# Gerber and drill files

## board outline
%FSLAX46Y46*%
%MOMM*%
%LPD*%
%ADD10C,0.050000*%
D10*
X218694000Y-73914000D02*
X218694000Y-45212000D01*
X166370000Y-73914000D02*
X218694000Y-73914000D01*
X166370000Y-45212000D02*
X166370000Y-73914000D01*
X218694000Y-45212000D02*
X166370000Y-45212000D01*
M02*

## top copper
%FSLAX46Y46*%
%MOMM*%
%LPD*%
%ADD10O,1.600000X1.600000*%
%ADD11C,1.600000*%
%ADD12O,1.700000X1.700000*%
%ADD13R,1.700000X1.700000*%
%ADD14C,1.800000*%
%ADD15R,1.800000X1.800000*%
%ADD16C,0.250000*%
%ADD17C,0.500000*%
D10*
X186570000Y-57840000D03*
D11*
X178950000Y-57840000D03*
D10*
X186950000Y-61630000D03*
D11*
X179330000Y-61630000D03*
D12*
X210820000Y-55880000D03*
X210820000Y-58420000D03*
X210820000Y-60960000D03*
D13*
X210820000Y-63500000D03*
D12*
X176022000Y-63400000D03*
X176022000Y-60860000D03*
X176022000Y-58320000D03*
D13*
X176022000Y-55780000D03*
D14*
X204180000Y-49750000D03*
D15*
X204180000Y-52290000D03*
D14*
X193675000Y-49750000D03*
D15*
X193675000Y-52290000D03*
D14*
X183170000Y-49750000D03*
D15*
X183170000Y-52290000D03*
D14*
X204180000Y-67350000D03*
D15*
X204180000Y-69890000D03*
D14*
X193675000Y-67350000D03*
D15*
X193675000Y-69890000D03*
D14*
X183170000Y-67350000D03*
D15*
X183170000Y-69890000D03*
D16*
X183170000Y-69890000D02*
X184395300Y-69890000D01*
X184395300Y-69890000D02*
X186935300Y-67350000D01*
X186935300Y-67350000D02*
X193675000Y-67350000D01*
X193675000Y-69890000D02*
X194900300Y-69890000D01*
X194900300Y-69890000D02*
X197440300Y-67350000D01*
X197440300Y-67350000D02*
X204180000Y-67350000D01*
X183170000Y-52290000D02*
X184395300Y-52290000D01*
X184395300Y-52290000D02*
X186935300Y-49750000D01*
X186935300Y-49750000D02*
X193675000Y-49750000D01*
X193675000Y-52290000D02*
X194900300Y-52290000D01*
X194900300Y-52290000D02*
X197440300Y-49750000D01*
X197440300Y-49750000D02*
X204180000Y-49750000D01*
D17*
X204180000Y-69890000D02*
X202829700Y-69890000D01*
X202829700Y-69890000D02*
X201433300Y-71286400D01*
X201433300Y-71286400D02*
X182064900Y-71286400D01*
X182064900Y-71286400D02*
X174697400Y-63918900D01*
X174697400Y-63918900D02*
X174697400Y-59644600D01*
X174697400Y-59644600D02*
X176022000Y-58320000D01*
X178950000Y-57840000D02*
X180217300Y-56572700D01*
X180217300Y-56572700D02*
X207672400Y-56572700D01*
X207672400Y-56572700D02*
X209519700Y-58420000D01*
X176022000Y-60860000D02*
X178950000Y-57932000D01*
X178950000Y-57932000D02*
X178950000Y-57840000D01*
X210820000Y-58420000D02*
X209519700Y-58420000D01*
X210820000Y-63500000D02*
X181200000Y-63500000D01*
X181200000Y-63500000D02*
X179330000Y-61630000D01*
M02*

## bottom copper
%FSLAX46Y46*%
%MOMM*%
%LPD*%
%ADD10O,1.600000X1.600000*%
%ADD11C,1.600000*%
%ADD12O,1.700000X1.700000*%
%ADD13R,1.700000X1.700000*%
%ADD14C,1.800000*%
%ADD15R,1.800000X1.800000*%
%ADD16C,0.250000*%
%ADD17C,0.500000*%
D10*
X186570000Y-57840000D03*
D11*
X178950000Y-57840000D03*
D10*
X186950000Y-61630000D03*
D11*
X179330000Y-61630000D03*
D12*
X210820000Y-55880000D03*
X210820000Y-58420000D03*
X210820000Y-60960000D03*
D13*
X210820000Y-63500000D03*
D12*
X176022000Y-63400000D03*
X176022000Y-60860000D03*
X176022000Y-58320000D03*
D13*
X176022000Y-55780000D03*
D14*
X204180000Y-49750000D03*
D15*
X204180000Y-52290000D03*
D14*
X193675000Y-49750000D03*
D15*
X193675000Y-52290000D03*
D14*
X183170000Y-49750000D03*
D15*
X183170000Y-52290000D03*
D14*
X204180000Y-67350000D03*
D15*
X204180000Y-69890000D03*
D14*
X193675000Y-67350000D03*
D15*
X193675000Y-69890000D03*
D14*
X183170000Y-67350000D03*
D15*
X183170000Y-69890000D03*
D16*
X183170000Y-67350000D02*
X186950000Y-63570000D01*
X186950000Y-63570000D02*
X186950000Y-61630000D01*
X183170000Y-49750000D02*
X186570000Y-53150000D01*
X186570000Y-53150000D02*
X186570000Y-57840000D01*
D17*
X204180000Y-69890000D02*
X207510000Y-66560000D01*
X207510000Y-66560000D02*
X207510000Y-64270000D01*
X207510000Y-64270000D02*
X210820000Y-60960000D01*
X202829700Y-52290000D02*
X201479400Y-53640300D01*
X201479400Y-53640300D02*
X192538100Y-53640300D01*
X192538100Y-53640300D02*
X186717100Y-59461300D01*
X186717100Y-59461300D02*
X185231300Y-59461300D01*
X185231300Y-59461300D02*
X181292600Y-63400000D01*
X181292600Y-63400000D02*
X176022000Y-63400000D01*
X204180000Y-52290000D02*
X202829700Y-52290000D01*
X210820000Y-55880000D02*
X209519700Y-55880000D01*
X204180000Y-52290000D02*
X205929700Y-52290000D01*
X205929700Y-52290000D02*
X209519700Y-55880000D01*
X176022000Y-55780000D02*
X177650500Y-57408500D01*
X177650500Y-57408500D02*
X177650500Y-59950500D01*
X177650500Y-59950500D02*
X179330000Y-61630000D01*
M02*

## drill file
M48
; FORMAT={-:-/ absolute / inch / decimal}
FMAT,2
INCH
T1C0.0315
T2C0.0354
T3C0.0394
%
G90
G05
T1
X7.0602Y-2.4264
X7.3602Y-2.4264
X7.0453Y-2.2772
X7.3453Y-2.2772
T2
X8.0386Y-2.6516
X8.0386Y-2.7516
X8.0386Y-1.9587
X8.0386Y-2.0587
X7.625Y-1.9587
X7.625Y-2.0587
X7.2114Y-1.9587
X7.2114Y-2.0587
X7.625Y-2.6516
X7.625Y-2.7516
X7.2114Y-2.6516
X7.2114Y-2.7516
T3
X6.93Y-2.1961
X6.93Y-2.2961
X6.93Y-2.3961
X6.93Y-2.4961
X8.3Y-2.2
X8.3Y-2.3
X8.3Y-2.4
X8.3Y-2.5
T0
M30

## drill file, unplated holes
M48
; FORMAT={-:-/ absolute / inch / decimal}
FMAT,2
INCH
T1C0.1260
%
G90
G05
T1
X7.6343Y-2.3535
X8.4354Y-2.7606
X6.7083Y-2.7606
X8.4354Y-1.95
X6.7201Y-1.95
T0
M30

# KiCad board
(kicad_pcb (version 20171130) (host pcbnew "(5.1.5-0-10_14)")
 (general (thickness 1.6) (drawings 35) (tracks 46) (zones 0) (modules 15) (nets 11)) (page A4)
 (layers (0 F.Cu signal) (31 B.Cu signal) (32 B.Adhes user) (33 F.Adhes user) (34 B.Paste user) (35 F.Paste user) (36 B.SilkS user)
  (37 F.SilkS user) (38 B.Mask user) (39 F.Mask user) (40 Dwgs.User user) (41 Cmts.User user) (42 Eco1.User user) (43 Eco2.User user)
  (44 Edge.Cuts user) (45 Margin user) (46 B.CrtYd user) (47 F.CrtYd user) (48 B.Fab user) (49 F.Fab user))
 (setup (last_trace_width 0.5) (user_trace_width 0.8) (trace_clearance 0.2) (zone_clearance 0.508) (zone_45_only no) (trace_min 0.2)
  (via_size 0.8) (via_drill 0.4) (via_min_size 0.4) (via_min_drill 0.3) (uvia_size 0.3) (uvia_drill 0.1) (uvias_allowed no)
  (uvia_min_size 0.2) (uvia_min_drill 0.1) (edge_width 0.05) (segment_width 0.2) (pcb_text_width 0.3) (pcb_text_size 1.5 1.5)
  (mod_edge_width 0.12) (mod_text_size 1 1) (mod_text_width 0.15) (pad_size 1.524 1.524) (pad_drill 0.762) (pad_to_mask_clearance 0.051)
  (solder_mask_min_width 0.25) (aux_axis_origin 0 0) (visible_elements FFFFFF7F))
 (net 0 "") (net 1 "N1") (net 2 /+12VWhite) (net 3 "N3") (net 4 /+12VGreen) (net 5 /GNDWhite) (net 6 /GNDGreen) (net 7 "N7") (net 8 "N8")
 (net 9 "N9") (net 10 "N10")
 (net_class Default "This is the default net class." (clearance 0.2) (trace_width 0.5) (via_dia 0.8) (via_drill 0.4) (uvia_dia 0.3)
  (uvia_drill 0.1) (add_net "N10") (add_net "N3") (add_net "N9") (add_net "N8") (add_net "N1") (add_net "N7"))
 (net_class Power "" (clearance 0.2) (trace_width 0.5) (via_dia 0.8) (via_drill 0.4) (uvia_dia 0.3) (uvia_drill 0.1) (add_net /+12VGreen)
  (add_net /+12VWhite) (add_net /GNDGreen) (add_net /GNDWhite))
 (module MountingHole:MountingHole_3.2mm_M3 (layer F.Cu) (at 193.91 59.78)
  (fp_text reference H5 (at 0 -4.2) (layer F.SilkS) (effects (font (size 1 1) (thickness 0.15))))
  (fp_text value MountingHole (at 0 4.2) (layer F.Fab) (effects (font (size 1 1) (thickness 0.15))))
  (pad 1 np_thru_hole circle (at 0 0) (size 3.2 3.2) (drill 3.2) (layers *.Cu *.Mask)))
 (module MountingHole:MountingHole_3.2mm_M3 (layer F.Cu) (at 214.26 70.12)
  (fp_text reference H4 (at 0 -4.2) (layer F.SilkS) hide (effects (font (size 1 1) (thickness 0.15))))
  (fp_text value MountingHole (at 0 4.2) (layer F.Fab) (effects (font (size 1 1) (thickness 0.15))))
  (pad 1 np_thru_hole circle (at 0 0) (size 3.2 3.2) (drill 3.2) (layers *.Cu *.Mask)))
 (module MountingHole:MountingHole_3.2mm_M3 (layer F.Cu) (at 170.39 70.12)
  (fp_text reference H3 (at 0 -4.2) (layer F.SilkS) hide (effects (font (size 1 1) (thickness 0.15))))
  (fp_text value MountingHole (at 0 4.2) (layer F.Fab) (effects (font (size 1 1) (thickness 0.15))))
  (pad 1 np_thru_hole circle (at 0 0) (size 3.2 3.2) (drill 3.2) (layers *.Cu *.Mask)))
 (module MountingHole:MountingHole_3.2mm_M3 (layer F.Cu) (at 214.26 49.53)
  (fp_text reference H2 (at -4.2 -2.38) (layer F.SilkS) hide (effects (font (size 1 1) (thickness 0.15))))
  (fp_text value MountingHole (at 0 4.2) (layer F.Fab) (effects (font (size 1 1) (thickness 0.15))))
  (pad 1 np_thru_hole circle (at 0 0) (size 3.2 3.2) (drill 3.2) (layers *.Cu *.Mask)))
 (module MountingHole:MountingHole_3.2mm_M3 (layer F.Cu) (at 170.69 49.53)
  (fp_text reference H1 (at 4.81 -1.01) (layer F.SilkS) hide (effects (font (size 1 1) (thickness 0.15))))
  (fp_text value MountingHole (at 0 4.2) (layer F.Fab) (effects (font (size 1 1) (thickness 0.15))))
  (pad 1 np_thru_hole circle (at 0 0) (size 3.2 3.2) (drill 3.2) (layers *.Cu *.Mask)))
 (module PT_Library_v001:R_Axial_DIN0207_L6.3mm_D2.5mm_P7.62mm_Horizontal (layer B.Cu) (at 178.95 57.84)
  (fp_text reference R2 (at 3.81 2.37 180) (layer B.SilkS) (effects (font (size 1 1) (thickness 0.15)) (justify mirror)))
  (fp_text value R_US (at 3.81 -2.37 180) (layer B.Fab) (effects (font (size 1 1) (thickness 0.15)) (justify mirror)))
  (pad 2 thru_hole oval (at 7.62 0) (size 1.6 1.6) (drill 0.8) (layers *.Cu *.Mask) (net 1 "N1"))
  (pad 1 thru_hole circle (at 0 0) (size 1.6 1.6) (drill 0.8) (layers *.Cu *.Mask) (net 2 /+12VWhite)))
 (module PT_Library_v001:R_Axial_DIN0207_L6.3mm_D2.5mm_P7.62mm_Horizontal (layer B.Cu) (at 179.33 61.63)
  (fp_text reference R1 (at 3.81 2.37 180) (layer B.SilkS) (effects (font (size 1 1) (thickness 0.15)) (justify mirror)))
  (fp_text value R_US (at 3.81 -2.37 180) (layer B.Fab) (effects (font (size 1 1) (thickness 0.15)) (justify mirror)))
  (pad 2 thru_hole oval (at 7.62 0) (size 1.6 1.6) (drill 0.8) (layers *.Cu *.Mask) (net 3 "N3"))
  (pad 1 thru_hole circle (at 0 0) (size 1.6 1.6) (drill 0.8) (layers *.Cu *.Mask) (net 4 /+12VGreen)))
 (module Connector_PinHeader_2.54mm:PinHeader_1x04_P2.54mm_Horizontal (layer B.Cu) (at 210.82 63.5)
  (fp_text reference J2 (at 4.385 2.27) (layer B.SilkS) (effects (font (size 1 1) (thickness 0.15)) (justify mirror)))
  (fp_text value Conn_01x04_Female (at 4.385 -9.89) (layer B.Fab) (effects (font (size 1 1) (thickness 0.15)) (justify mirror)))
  (pad 4 thru_hole oval (at 0 -7.62) (size 1.7 1.7) (drill 1) (layers *.Cu *.Mask) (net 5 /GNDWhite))
  (pad 3 thru_hole oval (at 0 -5.08) (size 1.7 1.7) (drill 1) (layers *.Cu *.Mask) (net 2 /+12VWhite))
  (pad 2 thru_hole oval (at 0 -2.54) (size 1.7 1.7) (drill 1) (layers *.Cu *.Mask) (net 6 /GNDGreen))
  (pad 1 thru_hole rect (at 0 0) (size 1.7 1.7) (drill 1) (layers *.Cu *.Mask) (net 4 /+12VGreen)))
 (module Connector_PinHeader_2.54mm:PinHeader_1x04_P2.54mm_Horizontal (layer B.Cu) (at 176.022 55.78 180)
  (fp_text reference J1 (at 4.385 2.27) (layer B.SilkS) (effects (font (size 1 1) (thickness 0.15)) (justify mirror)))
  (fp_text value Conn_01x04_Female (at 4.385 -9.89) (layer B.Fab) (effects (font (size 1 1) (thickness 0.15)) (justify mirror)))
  (pad 4 thru_hole oval (at 0 -7.62 180) (size 1.7 1.7) (drill 1) (layers *.Cu *.Mask) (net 5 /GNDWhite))
  (pad 3 thru_hole oval (at 0 -5.08 180) (size 1.7 1.7) (drill 1) (layers *.Cu *.Mask) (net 2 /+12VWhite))
  (pad 2 thru_hole oval (at 0 -2.54 180) (size 1.7 1.7) (drill 1) (layers *.Cu *.Mask) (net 6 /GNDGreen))
  (pad 1 thru_hole rect (at 0 0 180) (size 1.7 1.7) (drill 1) (layers *.Cu *.Mask) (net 4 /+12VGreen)))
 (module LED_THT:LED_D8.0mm (layer F.Cu) (at 204.18 52.29 90)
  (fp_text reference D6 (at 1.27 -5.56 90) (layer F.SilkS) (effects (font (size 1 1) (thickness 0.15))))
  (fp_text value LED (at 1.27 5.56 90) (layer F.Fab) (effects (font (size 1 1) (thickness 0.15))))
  (pad 2 thru_hole circle (at 2.54 0 90) (size 1.8 1.8) (drill 0.9) (layers *.Cu *.Mask) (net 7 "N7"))
  (pad 1 thru_hole rect (at 0 0 90) (size 1.8 1.8) (drill 0.9) (layers *.Cu *.Mask) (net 5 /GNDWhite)))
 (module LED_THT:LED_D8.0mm (layer F.Cu) (at 193.675 52.29 90)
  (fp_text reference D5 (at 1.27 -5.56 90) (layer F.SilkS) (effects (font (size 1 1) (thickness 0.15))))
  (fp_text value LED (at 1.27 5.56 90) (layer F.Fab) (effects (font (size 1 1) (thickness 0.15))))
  (pad 2 thru_hole circle (at 2.54 0 90) (size 1.8 1.8) (drill 0.9) (layers *.Cu *.Mask) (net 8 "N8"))
  (pad 1 thru_hole rect (at 0 0 90) (size 1.8 1.8) (drill 0.9) (layers *.Cu *.Mask) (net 7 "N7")))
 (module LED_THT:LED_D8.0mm (layer F.Cu) (at 183.17 52.29 90)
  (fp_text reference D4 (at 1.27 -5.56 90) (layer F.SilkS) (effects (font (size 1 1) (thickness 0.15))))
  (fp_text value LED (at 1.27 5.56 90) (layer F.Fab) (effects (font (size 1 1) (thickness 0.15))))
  (pad 2 thru_hole circle (at 2.54 0 90) (size 1.8 1.8) (drill 0.9) (layers *.Cu *.Mask) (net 1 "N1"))
  (pad 1 thru_hole rect (at 0 0 90) (size 1.8 1.8) (drill 0.9) (layers *.Cu *.Mask) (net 8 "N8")))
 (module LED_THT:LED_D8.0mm (layer F.Cu) (at 204.18 69.89 90)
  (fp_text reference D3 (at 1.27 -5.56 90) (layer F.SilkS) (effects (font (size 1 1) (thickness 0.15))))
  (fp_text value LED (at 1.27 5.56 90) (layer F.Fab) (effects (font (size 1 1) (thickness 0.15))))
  (pad 2 thru_hole circle (at 2.54 0 90) (size 1.8 1.8) (drill 0.9) (layers *.Cu *.Mask) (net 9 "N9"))
  (pad 1 thru_hole rect (at 0 0 90) (size 1.8 1.8) (drill 0.9) (layers *.Cu *.Mask) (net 6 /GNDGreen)))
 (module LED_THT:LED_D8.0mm (layer F.Cu) (at 193.675 69.89 90)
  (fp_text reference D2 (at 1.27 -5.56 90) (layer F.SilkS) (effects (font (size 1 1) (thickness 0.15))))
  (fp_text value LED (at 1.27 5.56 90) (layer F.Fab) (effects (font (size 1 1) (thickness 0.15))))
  (pad 2 thru_hole circle (at 2.54 0 90) (size 1.8 1.8) (drill 0.9) (layers *.Cu *.Mask) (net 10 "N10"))
  (pad 1 thru_hole rect (at 0 0 90) (size 1.8 1.8) (drill 0.9) (layers *.Cu *.Mask) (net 9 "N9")))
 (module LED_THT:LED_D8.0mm (layer F.Cu) (at 183.17 69.89 90)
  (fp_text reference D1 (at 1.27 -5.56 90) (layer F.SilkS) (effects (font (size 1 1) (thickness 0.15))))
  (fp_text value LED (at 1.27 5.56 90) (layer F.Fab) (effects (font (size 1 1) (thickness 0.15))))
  (pad 2 thru_hole circle (at 2.54 0 90) (size 1.8 1.8) (drill 0.9) (layers *.Cu *.Mask) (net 3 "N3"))
  (pad 1 thru_hole rect (at 0 0 90) (size 1.8 1.8) (drill 0.9) (layers *.Cu *.Mask) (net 10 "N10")))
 (gr_line (start 218.694 73.914) (end 218.694 45.212) (layer Edge.Cuts) (width 0.05))
 (gr_line (start 166.37 73.914) (end 218.694 73.914) (layer Edge.Cuts) (width 0.05))
 (gr_line (start 166.37 45.212) (end 166.37 73.914) (layer Edge.Cuts) (width 0.05))
 (gr_line (start 218.694 45.212) (end 166.37 45.212) (layer Edge.Cuts) (width 0.05))
 (segment (start 183.17 69.89) (end 184.3953 69.89) (width 0.25) (layer F.Cu) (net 10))
 (segment (start 184.3953 69.89) (end 186.9353 67.35) (width 0.25) (layer F.Cu) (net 10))
 (segment (start 186.9353 67.35) (end 193.675 67.35) (width 0.25) (layer F.Cu) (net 10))
 (segment (start 183.17 67.35) (end 186.95 63.57) (width 0.25) (layer B.Cu) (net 3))
 (segment (start 186.95 63.57) (end 186.95 61.63) (width 0.25) (layer B.Cu) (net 3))
 (segment (start 193.675 69.89) (end 194.9003 69.89) (width 0.25) (layer F.Cu) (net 9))
 (segment (start 194.9003 69.89) (end 197.4403 67.35) (width 0.25) (layer F.Cu) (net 9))
 (segment (start 197.4403 67.35) (end 204.18 67.35) (width 0.25) (layer F.Cu) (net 9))
 (segment (start 183.17 49.75) (end 186.57 53.15) (width 0.25) (layer B.Cu) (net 1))
 (segment (start 186.57 53.15) (end 186.57 57.84) (width 0.25) (layer B.Cu) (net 1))
 (segment (start 183.17 52.29) (end 184.3953 52.29) (width 0.25) (layer F.Cu) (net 8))
 (segment (start 184.3953 52.29) (end 186.9353 49.75) (width 0.25) (layer F.Cu) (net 8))
 (segment (start 186.9353 49.75) (end 193.675 49.75) (width 0.25) (layer F.Cu) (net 8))
 (segment (start 193.675 52.29) (end 194.9003 52.29) (width 0.25) (layer F.Cu) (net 7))
 (segment (start 194.9003 52.29) (end 197.4403 49.75) (width 0.25) (layer F.Cu) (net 7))
 (segment (start 197.4403 49.75) (end 204.18 49.75) (width 0.25) (layer F.Cu) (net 7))
 (segment (start 204.18 69.89) (end 202.8297 69.89) (width 0.5) (layer F.Cu) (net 6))
 (segment (start 202.8297 69.89) (end 201.4333 71.2864) (width 0.5) (layer F.Cu) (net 6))
 (segment (start 201.4333 71.2864) (end 182.0649 71.2864) (width 0.5) (layer F.Cu) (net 6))
 (segment (start 182.0649 71.2864) (end 174.6974 63.9189) (width 0.5) (layer F.Cu) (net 6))
 (segment (start 174.6974 63.9189) (end 174.6974 59.6446) (width 0.5) (layer F.Cu) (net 6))
 (segment (start 174.6974 59.6446) (end 176.022 58.32) (width 0.5) (layer F.Cu) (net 6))
 (segment (start 204.18 69.89) (end 207.51 66.56) (width 0.5) (layer B.Cu) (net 6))
 (segment (start 207.51 66.56) (end 207.51 64.27) (width 0.5) (layer B.Cu) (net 6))
 (segment (start 207.51 64.27) (end 210.82 60.96) (width 0.5) (layer B.Cu) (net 6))
 (segment (start 202.8297 52.29) (end 201.4794 53.6403) (width 0.5) (layer B.Cu) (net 5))
 (segment (start 201.4794 53.6403) (end 192.5381 53.6403) (width 0.5) (layer B.Cu) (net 5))
 (segment (start 192.5381 53.6403) (end 186.7171 59.4613) (width 0.5) (layer B.Cu) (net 5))
 (segment (start 186.7171 59.4613) (end 185.2313 59.4613) (width 0.5) (layer B.Cu) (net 5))
 (segment (start 185.2313 59.4613) (end 181.2926 63.4) (width 0.5) (layer B.Cu) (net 5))
 (segment (start 181.2926 63.4) (end 176.022 63.4) (width 0.5) (layer B.Cu) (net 5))
 (segment (start 204.18 52.29) (end 202.8297 52.29) (width 0.5) (layer B.Cu) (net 5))
 (segment (start 210.82 55.88) (end 209.5197 55.88) (width 0.5) (layer B.Cu) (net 5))
 (segment (start 204.18 52.29) (end 205.9297 52.29) (width 0.5) (layer B.Cu) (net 5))
 (segment (start 205.9297 52.29) (end 209.5197 55.88) (width 0.5) (layer B.Cu) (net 5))
 (segment (start 178.95 57.84) (end 180.2173 56.5727) (width 0.5) (layer F.Cu) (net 2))
 (segment (start 180.2173 56.5727) (end 207.6724 56.5727) (width 0.5) (layer F.Cu) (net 2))
 (segment (start 207.6724 56.5727) (end 209.5197 58.42) (width 0.5) (layer F.Cu) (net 2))
 (segment (start 176.022 60.86) (end 178.95 57.932) (width 0.5) (layer F.Cu) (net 2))
 (segment (start 178.95 57.932) (end 178.95 57.84) (width 0.5) (layer F.Cu) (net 2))
 (segment (start 210.82 58.42) (end 209.5197 58.42) (width 0.5) (layer F.Cu) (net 2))
 (segment (start 210.82 63.5) (end 181.2 63.5) (width 0.5) (layer F.Cu) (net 4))
 (segment (start 181.2 63.5) (end 179.33 61.63) (width 0.5) (layer F.Cu) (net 4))
 (segment (start 176.022 55.78) (end 177.6505 57.4085) (width 0.5) (layer B.Cu) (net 4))
 (segment (start 177.6505 57.4085) (end 177.6505 59.9505) (width 0.5) (layer B.Cu) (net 4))
 (segment (start 177.6505 59.9505) (end 179.33 61.63) (width 0.5) (layer B.Cu) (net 4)))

